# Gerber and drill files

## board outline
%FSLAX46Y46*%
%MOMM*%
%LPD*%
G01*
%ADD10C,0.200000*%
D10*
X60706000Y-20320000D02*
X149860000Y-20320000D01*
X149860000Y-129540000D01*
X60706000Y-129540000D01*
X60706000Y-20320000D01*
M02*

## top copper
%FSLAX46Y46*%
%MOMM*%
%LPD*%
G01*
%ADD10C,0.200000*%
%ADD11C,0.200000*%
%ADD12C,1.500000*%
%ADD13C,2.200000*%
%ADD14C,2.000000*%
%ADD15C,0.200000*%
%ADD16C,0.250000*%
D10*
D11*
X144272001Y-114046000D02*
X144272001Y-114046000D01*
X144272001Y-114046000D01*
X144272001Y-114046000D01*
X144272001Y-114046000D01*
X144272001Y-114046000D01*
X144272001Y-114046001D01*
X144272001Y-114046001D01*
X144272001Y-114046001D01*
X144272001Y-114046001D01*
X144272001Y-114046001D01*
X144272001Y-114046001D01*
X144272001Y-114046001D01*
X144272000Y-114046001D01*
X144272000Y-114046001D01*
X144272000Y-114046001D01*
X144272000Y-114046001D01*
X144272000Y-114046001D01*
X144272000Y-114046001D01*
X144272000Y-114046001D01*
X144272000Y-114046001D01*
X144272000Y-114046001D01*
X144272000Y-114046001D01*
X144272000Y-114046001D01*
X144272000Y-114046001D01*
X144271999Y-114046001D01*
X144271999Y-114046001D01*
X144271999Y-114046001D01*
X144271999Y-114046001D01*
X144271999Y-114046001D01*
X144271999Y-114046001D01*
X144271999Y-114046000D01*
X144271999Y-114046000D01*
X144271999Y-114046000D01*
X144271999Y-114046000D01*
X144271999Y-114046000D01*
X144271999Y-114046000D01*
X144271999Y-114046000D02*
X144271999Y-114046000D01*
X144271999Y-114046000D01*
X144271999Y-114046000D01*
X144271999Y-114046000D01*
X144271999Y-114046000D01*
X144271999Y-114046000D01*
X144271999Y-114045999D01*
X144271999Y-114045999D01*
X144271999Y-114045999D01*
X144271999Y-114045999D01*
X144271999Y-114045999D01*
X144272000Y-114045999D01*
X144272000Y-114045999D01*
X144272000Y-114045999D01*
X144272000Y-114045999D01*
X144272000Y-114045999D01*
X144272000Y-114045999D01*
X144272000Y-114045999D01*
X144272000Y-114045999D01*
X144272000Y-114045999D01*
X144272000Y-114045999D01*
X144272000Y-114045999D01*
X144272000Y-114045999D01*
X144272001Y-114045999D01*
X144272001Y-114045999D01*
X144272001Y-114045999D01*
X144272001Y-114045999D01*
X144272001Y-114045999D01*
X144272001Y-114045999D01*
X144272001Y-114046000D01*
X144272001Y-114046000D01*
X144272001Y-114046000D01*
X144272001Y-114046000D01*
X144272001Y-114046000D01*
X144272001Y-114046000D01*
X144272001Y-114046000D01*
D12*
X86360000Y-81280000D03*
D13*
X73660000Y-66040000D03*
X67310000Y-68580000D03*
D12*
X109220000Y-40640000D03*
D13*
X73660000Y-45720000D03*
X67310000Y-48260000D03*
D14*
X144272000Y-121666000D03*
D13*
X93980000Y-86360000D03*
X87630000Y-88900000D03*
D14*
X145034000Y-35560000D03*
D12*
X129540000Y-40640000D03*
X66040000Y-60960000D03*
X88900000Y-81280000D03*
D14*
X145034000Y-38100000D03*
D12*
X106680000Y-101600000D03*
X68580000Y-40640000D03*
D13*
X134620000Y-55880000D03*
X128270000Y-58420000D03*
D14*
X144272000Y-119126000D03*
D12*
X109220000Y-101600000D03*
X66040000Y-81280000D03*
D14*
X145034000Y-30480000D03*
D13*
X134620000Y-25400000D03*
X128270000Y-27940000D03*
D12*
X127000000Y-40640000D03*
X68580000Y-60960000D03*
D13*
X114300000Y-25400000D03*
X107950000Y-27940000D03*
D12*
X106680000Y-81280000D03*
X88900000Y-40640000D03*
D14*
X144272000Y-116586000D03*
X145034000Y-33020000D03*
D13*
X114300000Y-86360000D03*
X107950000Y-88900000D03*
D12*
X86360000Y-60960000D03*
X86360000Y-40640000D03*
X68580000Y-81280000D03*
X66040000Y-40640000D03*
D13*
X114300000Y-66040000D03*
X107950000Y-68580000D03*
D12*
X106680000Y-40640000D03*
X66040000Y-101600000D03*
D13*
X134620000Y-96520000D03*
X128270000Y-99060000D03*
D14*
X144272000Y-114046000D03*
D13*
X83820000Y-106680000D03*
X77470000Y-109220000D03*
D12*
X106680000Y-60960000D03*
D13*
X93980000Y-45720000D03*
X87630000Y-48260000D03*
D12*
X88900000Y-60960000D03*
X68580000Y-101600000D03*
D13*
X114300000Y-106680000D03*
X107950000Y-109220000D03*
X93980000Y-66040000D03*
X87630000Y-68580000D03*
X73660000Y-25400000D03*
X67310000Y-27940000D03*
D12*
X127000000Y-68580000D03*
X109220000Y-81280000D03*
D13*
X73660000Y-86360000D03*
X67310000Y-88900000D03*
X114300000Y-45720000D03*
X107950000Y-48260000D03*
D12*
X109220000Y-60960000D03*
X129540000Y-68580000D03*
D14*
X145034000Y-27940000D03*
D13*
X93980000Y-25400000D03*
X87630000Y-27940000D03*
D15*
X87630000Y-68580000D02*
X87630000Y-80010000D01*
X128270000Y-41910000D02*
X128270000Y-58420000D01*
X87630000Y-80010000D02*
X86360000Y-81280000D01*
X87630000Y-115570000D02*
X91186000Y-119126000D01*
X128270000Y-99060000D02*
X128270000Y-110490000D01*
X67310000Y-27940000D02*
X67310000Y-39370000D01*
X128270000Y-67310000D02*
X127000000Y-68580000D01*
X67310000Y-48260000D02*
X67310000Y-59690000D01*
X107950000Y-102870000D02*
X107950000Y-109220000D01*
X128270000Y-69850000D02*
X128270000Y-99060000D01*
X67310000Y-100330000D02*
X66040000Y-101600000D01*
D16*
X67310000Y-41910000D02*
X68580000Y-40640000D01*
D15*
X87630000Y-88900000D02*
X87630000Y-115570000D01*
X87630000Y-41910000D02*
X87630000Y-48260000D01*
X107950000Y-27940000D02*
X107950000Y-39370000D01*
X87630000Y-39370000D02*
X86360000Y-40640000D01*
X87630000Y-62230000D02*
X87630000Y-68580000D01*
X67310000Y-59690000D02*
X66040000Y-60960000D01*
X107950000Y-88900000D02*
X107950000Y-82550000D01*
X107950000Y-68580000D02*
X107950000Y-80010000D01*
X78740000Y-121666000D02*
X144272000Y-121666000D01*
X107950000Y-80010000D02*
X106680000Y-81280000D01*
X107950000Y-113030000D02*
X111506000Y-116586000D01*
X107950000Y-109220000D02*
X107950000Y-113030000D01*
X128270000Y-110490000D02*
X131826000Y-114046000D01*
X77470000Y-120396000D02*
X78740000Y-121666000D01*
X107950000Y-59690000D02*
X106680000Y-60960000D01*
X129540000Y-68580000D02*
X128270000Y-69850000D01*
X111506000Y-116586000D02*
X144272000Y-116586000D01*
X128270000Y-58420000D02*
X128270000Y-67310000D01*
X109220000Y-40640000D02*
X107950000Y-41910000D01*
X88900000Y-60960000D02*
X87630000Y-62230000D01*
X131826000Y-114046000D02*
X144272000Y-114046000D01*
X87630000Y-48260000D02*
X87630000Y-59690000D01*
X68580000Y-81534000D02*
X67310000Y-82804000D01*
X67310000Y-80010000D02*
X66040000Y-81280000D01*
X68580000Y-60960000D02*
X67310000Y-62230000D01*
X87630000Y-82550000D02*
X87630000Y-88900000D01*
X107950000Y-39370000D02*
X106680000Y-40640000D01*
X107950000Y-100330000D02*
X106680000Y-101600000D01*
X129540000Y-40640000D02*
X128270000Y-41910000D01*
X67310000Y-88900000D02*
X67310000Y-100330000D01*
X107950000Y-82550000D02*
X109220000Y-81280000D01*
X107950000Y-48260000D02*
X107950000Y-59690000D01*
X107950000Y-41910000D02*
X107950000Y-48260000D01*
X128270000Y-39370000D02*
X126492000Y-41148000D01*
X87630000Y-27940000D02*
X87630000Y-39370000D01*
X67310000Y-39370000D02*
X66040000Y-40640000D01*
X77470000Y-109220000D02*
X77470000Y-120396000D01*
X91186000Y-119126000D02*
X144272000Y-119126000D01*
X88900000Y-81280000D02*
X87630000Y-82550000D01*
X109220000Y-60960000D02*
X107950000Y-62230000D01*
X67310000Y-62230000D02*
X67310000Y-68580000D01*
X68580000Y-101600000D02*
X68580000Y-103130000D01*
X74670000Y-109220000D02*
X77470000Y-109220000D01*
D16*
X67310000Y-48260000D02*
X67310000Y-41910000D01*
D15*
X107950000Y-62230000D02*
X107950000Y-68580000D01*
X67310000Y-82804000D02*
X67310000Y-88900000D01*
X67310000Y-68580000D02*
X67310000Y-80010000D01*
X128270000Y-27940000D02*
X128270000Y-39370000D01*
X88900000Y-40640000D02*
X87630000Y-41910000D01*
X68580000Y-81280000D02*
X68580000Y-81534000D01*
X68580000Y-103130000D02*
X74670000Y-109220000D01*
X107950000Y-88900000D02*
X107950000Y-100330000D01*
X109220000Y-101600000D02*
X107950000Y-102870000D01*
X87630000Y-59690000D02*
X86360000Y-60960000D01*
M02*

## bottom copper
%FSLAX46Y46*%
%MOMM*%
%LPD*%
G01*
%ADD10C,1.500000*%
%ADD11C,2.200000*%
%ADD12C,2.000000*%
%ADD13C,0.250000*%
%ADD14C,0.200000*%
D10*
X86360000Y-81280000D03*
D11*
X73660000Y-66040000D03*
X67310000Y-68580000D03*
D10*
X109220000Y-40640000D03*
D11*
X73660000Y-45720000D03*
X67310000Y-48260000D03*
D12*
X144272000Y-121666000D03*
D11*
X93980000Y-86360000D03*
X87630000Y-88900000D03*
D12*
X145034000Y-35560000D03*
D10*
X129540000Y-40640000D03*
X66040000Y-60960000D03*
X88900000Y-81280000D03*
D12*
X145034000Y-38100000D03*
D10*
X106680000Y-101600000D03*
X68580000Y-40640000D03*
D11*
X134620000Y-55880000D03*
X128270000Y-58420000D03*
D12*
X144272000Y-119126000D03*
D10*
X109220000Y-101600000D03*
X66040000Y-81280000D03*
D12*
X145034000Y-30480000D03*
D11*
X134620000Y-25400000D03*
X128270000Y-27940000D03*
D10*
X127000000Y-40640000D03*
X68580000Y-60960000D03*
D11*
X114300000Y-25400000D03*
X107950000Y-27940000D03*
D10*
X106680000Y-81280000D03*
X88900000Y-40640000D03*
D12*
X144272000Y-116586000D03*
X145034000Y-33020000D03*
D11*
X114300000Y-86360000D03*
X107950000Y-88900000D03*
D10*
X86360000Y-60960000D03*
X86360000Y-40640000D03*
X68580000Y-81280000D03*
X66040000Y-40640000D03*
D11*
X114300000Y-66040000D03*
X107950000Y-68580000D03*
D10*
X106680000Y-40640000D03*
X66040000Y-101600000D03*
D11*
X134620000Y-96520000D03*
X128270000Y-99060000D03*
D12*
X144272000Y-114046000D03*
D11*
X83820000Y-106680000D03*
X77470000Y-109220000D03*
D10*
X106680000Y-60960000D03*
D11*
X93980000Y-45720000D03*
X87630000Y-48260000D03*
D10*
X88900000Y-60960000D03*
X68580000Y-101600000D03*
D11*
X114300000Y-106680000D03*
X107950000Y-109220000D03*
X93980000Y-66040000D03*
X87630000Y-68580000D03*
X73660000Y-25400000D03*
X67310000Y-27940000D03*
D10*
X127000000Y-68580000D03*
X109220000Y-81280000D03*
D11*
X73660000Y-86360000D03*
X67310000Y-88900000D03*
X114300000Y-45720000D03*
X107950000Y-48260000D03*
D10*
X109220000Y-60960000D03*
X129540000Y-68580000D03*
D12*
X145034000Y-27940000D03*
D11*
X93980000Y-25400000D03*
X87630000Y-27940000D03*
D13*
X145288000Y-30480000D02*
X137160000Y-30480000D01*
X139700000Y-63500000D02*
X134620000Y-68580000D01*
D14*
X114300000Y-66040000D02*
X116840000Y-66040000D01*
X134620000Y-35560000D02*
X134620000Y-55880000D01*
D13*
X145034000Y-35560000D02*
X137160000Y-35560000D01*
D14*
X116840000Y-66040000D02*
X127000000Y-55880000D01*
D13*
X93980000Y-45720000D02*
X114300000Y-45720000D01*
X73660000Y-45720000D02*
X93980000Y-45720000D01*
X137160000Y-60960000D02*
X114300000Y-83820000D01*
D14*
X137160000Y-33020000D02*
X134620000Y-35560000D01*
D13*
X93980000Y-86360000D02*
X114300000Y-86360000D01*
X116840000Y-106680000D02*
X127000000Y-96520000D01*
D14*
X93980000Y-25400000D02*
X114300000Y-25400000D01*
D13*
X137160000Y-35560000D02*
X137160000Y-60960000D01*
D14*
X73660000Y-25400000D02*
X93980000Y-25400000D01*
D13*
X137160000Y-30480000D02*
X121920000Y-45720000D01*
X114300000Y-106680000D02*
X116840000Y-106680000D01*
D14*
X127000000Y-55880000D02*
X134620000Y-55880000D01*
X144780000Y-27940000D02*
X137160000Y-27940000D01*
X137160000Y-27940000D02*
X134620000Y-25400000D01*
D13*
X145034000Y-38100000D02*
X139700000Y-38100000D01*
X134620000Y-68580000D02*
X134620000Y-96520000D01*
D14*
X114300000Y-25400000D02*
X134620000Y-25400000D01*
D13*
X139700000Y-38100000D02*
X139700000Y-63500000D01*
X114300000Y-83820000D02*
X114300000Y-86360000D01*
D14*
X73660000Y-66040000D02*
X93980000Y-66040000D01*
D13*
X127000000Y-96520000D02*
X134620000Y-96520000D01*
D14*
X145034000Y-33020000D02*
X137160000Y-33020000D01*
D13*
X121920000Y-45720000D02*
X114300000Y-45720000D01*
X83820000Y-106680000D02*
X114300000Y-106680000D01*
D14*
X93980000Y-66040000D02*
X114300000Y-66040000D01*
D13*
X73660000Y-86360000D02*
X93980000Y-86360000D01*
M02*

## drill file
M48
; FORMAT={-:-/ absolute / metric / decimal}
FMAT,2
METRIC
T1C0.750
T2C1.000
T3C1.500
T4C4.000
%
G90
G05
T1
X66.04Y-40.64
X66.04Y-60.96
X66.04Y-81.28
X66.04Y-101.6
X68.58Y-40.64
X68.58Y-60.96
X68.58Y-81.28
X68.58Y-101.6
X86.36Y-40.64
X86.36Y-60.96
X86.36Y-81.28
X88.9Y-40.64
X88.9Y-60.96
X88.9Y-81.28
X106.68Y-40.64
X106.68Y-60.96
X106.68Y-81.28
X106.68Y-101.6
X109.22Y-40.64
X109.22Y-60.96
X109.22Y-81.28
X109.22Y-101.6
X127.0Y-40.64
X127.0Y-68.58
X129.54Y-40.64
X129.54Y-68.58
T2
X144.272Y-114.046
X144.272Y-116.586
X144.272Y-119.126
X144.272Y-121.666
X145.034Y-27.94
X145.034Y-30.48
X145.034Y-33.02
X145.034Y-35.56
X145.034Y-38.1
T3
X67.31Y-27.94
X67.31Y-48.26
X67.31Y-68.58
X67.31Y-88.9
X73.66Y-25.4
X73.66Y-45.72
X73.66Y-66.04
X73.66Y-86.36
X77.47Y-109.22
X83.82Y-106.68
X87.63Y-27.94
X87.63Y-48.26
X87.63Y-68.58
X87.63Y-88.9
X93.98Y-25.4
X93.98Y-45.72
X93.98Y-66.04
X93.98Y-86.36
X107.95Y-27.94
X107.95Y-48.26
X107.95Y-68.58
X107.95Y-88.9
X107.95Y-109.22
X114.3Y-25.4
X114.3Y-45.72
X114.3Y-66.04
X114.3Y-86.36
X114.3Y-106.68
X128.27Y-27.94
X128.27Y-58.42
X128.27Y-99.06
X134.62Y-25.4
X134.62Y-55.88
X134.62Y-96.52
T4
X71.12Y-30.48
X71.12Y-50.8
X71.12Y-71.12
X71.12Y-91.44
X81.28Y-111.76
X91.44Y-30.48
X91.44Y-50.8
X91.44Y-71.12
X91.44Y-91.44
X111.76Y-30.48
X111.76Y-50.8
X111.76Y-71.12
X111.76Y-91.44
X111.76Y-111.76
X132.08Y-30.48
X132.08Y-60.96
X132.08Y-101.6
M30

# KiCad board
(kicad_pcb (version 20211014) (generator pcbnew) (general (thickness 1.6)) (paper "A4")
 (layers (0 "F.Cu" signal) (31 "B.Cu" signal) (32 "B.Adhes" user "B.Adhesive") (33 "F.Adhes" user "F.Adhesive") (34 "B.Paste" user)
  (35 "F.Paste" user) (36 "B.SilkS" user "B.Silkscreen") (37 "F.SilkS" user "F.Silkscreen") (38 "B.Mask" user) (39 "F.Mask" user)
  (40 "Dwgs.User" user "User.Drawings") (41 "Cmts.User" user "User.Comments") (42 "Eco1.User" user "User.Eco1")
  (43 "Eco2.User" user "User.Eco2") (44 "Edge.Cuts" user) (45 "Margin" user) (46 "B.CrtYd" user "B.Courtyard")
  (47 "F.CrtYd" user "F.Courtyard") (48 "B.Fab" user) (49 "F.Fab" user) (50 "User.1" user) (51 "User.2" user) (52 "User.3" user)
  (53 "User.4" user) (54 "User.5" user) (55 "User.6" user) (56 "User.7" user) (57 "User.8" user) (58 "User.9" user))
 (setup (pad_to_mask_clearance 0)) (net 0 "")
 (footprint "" (layer "F.Cu") (at 86.36 81.28)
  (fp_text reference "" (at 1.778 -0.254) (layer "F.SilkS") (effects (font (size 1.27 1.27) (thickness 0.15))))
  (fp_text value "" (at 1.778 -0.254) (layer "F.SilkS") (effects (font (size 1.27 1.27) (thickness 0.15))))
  (pad "1" thru_hole circle (at 0 0) (size 1.5 1.5) (drill 0.75) (layers *.Cu *.Mask)))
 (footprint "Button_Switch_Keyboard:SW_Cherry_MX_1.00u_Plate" (layer "F.Cu") (at 73.66 66.04)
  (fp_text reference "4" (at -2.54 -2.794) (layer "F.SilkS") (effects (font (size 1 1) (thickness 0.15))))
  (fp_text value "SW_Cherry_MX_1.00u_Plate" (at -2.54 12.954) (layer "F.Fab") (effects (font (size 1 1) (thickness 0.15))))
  (pad "" np_thru_hole circle (at -2.54 5.08) (size 4 4) (drill 4) (layers *.Cu *.Mask))
  (pad "1" thru_hole circle (at 0 0) (size 2.2 2.2) (drill 1.5) (layers *.Cu *.Mask))
  (pad "2" thru_hole circle (at -6.35 2.54) (size 2.2 2.2) (drill 1.5) (layers *.Cu *.Mask)))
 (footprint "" (layer "F.Cu") (at 109.22 40.64)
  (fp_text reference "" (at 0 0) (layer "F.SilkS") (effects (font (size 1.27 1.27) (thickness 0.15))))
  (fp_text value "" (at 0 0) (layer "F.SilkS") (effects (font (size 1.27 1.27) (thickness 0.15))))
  (pad "1" thru_hole circle (at 0 0) (size 1.5 1.5) (drill 0.75) (layers *.Cu *.Mask)))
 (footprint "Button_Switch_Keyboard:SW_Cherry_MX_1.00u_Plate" (layer "F.Cu") (at 73.66 45.72)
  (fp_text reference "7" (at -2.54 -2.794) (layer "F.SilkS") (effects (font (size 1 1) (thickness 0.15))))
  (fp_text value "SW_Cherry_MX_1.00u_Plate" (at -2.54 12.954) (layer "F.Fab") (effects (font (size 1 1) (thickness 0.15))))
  (pad "" np_thru_hole circle (at -2.54 5.08) (size 4 4) (drill 4) (layers *.Cu *.Mask))
  (pad "1" thru_hole circle (at 0 0) (size 2.2 2.2) (drill 1.5) (layers *.Cu *.Mask))
  (pad "2" thru_hole circle (at -6.35 2.54) (size 2.2 2.2) (drill 1.5) (layers *.Cu *.Mask)))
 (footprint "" (layer "F.Cu") (at 144.272 121.666)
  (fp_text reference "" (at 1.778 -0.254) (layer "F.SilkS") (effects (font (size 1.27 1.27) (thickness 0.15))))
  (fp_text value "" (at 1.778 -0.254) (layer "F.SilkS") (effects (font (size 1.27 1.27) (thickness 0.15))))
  (pad "1" thru_hole circle (at 0 0) (size 2 2) (drill 1) (layers *.Cu *.Mask)))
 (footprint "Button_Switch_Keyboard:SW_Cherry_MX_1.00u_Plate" (layer "F.Cu") (at 93.98 86.36)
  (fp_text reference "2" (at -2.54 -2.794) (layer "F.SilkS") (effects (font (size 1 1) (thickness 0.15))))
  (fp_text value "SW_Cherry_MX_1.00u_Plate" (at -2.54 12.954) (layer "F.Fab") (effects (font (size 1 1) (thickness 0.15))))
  (pad "" np_thru_hole circle (at -2.54 5.08) (size 4 4) (drill 4) (layers *.Cu *.Mask))
  (pad "1" thru_hole circle (at 0 0) (size 2.2 2.2) (drill 1.5) (layers *.Cu *.Mask))
  (pad "2" thru_hole circle (at -6.35 2.54) (size 2.2 2.2) (drill 1.5) (layers *.Cu *.Mask)))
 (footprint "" (layer "F.Cu") (at 145.034 35.56)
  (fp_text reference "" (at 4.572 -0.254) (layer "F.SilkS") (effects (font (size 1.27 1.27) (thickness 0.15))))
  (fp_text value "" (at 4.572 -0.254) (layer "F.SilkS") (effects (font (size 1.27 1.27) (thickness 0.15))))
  (pad "1" thru_hole circle (at 0 0) (size 2 2) (drill 1) (layers *.Cu *.Mask)))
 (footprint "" (layer "F.Cu") (at 129.54 40.64)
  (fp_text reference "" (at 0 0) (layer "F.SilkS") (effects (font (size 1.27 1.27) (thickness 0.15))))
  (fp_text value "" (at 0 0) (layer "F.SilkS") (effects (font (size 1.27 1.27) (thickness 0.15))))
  (pad "1" thru_hole circle (at 0 0) (size 1.5 1.5) (drill 0.75) (layers *.Cu *.Mask)))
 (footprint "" (layer "F.Cu") (at 66.04 60.96)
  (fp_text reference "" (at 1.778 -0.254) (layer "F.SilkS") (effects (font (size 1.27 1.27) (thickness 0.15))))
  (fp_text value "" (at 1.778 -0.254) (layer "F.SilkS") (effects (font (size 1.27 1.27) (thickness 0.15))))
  (pad "1" thru_hole circle (at 0 0) (size 1.5 1.5) (drill 0.75) (layers *.Cu *.Mask)))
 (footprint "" (layer "F.Cu") (at 88.9 81.28)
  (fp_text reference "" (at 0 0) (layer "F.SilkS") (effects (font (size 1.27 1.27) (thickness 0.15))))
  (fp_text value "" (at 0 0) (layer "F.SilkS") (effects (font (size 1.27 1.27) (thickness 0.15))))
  (pad "1" thru_hole circle (at 0 0) (size 1.5 1.5) (drill 0.75) (layers *.Cu *.Mask)))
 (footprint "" (layer "F.Cu") (at 145.034 38.1)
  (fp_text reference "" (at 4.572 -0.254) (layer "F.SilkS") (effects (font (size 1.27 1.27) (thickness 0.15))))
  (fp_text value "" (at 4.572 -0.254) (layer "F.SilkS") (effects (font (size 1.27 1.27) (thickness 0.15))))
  (pad "1" thru_hole circle (at 0 0) (size 2 2) (drill 1) (layers *.Cu *.Mask)))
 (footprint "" (layer "F.Cu") (at 106.68 101.6)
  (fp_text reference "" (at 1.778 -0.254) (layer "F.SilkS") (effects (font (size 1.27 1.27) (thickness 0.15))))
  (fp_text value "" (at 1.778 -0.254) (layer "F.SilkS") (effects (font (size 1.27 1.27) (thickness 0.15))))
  (pad "1" thru_hole circle (at 0 0) (size 1.5 1.5) (drill 0.75) (layers *.Cu *.Mask)))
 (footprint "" (layer "F.Cu") (at 68.58 40.64)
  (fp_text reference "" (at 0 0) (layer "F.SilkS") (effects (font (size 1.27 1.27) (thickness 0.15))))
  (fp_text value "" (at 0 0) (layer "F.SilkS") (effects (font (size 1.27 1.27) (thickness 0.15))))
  (pad "1" thru_hole circle (at 0 0) (size 1.5 1.5) (drill 0.75) (layers *.Cu *.Mask)))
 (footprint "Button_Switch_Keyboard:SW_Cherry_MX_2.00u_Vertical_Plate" (layer "F.Cu") (at 134.62 55.88)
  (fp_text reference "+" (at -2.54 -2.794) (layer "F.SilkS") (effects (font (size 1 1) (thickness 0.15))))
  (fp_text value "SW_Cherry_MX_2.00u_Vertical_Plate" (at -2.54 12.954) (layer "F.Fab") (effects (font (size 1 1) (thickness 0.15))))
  (pad "" np_thru_hole circle (at -2.54 5.08) (size 4 4) (drill 4) (layers *.Cu *.Mask))
  (pad "1" thru_hole circle (at 0 0) (size 2.2 2.2) (drill 1.5) (layers *.Cu *.Mask))
  (pad "2" thru_hole circle (at -6.35 2.54) (size 2.2 2.2) (drill 1.5) (layers *.Cu *.Mask)))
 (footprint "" (layer "F.Cu") (at 144.272 119.126)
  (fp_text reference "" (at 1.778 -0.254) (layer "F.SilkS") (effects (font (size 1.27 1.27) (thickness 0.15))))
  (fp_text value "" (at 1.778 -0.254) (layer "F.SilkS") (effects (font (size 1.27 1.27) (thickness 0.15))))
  (pad "1" thru_hole circle (at 0 0) (size 2 2) (drill 1) (layers *.Cu *.Mask)))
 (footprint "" (layer "F.Cu") (at 109.22 101.6)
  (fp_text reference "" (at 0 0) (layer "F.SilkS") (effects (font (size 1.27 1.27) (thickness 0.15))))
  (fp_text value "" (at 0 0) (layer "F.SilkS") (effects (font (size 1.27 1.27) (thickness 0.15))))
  (pad "1" thru_hole circle (at 0 0) (size 1.5 1.5) (drill 0.75) (layers *.Cu *.Mask)))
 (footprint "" (layer "F.Cu") (at 66.04 81.28)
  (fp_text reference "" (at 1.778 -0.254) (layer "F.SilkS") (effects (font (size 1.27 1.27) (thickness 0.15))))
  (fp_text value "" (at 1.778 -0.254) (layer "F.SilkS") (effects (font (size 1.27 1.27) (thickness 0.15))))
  (pad "1" thru_hole circle (at 0 0) (size 1.5 1.5) (drill 0.75) (layers *.Cu *.Mask)))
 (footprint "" (layer "F.Cu") (at 145.034 30.48)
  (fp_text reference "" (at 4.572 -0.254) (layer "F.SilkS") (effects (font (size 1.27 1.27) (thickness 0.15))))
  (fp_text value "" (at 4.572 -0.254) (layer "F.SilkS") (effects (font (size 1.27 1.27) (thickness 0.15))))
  (pad "1" thru_hole circle (at 0 0) (size 2 2) (drill 1) (layers *.Cu *.Mask)))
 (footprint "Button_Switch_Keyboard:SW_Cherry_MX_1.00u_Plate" (layer "F.Cu") (at 134.62 25.4)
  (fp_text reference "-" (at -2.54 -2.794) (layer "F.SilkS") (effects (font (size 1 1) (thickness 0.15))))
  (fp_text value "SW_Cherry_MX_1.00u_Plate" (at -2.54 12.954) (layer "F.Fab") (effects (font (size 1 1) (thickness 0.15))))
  (pad "" np_thru_hole circle (at -2.54 5.08) (size 4 4) (drill 4) (layers *.Cu *.Mask))
  (pad "1" thru_hole circle (at 0 0) (size 2.2 2.2) (drill 1.5) (layers *.Cu *.Mask))
  (pad "2" thru_hole circle (at -6.35 2.54) (size 2.2 2.2) (drill 1.5) (layers *.Cu *.Mask)))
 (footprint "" (layer "F.Cu") (at 127 40.64)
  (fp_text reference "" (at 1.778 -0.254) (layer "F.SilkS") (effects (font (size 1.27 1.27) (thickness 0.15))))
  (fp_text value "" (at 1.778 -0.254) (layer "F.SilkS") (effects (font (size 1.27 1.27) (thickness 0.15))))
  (pad "1" thru_hole circle (at 0 0) (size 1.5 1.5) (drill 0.75) (layers *.Cu *.Mask)))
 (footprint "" (layer "F.Cu") (at 68.58 60.96)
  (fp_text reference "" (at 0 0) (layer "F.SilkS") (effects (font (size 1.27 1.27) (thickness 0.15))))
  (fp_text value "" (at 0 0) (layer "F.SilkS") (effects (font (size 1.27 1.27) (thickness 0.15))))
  (pad "1" thru_hole circle (at 0 0) (size 1.5 1.5) (drill 0.75) (layers *.Cu *.Mask)))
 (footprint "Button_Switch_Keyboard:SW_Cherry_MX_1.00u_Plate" (layer "F.Cu") (at 114.3 25.4)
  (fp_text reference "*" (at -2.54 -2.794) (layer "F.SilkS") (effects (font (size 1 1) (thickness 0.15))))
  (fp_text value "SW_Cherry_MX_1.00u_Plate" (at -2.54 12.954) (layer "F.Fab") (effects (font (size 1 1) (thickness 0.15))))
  (pad "" np_thru_hole circle (at -2.54 5.08) (size 4 4) (drill 4) (layers *.Cu *.Mask))
  (pad "1" thru_hole circle (at 0 0) (size 2.2 2.2) (drill 1.5) (layers *.Cu *.Mask))
  (pad "2" thru_hole circle (at -6.35 2.54) (size 2.2 2.2) (drill 1.5) (layers *.Cu *.Mask)))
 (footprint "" (layer "F.Cu") (at 106.68 81.28)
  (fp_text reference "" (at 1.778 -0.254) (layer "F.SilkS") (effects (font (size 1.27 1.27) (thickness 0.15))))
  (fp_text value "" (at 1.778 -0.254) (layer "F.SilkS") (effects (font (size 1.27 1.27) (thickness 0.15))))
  (pad "1" thru_hole circle (at 0 0) (size 1.5 1.5) (drill 0.75) (layers *.Cu *.Mask)))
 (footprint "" (layer "F.Cu") (at 88.9 40.64)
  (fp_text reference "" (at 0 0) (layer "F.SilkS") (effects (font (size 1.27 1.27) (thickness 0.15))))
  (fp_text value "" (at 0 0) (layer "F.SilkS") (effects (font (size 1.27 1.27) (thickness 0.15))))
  (pad "1" thru_hole circle (at 0 0) (size 1.5 1.5) (drill 0.75) (layers *.Cu *.Mask)))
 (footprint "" (layer "F.Cu") (at 144.272 116.586)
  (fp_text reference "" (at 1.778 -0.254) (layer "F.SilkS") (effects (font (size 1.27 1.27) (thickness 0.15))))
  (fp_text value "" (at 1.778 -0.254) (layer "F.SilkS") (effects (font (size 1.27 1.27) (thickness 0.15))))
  (pad "1" thru_hole circle (at 0 0) (size 2 2) (drill 1) (layers *.Cu *.Mask)))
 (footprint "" (layer "F.Cu") (at 145.034 33.02)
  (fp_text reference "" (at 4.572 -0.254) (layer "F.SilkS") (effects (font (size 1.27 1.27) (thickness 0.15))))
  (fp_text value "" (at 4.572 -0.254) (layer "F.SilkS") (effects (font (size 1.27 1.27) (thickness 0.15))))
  (pad "1" thru_hole circle (at 0 0) (size 2 2) (drill 1) (layers *.Cu *.Mask)))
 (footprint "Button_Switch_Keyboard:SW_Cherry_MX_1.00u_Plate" (layer "F.Cu") (at 114.3 86.36)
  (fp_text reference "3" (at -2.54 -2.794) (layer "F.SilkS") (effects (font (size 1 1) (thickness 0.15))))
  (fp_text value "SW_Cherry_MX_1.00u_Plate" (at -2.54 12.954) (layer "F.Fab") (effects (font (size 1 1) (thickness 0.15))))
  (pad "" np_thru_hole circle (at -2.54 5.08) (size 4 4) (drill 4) (layers *.Cu *.Mask))
  (pad "1" thru_hole circle (at 0 0) (size 2.2 2.2) (drill 1.5) (layers *.Cu *.Mask))
  (pad "2" thru_hole circle (at -6.35 2.54) (size 2.2 2.2) (drill 1.5) (layers *.Cu *.Mask)))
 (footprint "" (layer "F.Cu") (at 86.36 60.96)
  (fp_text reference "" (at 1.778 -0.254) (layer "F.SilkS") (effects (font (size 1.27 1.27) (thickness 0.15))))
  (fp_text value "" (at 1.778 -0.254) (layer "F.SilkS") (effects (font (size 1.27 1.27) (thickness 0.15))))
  (pad "1" thru_hole circle (at 0 0) (size 1.5 1.5) (drill 0.75) (layers *.Cu *.Mask)))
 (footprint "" (layer "F.Cu") (at 86.36 40.64)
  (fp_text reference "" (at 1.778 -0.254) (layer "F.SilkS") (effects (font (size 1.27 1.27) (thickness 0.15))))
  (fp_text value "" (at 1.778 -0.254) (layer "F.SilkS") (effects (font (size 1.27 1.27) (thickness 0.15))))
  (pad "1" thru_hole circle (at 0 0) (size 1.5 1.5) (drill 0.75) (layers *.Cu *.Mask)))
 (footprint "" (layer "F.Cu") (at 68.58 81.28)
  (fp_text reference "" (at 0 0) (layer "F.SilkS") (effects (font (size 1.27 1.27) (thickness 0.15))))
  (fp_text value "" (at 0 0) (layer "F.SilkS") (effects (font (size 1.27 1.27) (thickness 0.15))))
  (pad "1" thru_hole circle (at 0 0) (size 1.5 1.5) (drill 0.75) (layers *.Cu *.Mask)))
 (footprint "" (layer "F.Cu") (at 66.04 40.64)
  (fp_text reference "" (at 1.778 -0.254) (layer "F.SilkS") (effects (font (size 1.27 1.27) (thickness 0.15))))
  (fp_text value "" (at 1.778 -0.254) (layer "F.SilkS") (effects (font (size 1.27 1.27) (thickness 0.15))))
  (pad "1" thru_hole circle (at 0 0) (size 1.5 1.5) (drill 0.75) (layers *.Cu *.Mask)))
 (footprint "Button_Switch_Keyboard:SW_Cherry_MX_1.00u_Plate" (layer "F.Cu") (at 114.3 66.04)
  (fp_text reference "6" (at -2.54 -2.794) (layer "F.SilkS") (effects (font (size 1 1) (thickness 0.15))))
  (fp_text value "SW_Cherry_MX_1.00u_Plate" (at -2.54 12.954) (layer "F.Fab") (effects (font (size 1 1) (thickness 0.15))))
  (pad "" np_thru_hole circle (at -2.54 5.08) (size 4 4) (drill 4) (layers *.Cu *.Mask))
  (pad "1" thru_hole circle (at 0 0) (size 2.2 2.2) (drill 1.5) (layers *.Cu *.Mask))
  (pad "2" thru_hole circle (at -6.35 2.54) (size 2.2 2.2) (drill 1.5) (layers *.Cu *.Mask)))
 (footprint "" (layer "F.Cu") (at 106.68 40.64)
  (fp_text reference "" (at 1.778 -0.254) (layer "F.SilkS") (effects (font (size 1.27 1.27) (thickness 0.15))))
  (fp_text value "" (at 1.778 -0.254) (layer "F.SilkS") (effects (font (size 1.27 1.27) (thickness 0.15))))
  (pad "1" thru_hole circle (at 0 0) (size 1.5 1.5) (drill 0.75) (layers *.Cu *.Mask)))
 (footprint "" (layer "F.Cu") (at 66.04 101.6)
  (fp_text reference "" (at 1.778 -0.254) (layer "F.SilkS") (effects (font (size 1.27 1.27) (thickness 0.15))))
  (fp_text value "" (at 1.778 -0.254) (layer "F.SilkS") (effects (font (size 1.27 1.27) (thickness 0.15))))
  (pad "1" thru_hole circle (at 0 0) (size 1.5 1.5) (drill 0.75) (layers *.Cu *.Mask)))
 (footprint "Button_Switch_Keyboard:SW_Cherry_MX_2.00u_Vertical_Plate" (layer "F.Cu") (at 134.62 96.52)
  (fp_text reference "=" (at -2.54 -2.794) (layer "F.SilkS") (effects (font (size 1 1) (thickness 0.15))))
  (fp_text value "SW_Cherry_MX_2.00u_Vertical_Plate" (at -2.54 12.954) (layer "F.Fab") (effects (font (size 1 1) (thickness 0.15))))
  (pad "" np_thru_hole circle (at -2.54 5.08) (size 4 4) (drill 4) (layers *.Cu *.Mask))
  (pad "1" thru_hole circle (at 0 0) (size 2.2 2.2) (drill 1.5) (layers *.Cu *.Mask))
  (pad "2" thru_hole circle (at -6.35 2.54) (size 2.2 2.2) (drill 1.5) (layers *.Cu *.Mask)))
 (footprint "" (layer "F.Cu") (at 144.272 114.046)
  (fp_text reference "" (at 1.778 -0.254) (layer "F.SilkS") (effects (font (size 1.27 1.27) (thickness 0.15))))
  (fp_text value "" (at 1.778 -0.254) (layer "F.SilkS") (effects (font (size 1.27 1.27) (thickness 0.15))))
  (pad "1" thru_hole circle (at 0 0) (size 2 2) (drill 1) (layers *.Cu *.Mask)))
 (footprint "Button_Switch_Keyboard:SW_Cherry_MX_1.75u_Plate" (layer "F.Cu") (at 83.82 106.68)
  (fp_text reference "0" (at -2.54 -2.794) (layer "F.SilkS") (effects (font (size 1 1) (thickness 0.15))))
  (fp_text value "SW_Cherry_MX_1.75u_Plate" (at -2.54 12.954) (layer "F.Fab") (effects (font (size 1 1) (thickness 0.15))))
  (pad "" np_thru_hole circle (at -2.54 5.08) (size 4 4) (drill 4) (layers *.Cu *.Mask))
  (pad "1" thru_hole circle (at 0 0) (size 2.2 2.2) (drill 1.5) (layers *.Cu *.Mask))
  (pad "2" thru_hole circle (at -6.35 2.54) (size 2.2 2.2) (drill 1.5) (layers *.Cu *.Mask)))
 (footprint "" (layer "F.Cu") (at 106.68 60.96)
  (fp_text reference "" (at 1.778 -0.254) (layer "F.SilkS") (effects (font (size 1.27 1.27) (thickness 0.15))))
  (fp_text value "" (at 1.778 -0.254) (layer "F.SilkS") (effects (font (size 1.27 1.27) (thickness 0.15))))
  (pad "1" thru_hole circle (at 0 0) (size 1.5 1.5) (drill 0.75) (layers *.Cu *.Mask)))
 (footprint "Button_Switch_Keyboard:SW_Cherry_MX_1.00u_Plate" (layer "F.Cu") (at 93.98 45.72)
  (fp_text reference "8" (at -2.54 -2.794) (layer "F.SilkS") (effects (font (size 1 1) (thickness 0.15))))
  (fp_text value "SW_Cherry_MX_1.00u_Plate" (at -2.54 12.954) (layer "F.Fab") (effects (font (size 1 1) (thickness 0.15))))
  (pad "" np_thru_hole circle (at -2.54 5.08) (size 4 4) (drill 4) (layers *.Cu *.Mask))
  (pad "1" thru_hole circle (at 0 0) (size 2.2 2.2) (drill 1.5) (layers *.Cu *.Mask))
  (pad "2" thru_hole circle (at -6.35 2.54) (size 2.2 2.2) (drill 1.5) (layers *.Cu *.Mask)))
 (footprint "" (layer "F.Cu") (at 88.9 60.96)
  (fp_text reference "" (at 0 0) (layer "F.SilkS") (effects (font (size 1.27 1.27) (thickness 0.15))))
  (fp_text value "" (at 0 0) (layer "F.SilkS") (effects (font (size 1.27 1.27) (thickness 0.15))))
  (pad "1" thru_hole circle (at 0 0) (size 1.5 1.5) (drill 0.75) (layers *.Cu *.Mask)))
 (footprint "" (layer "F.Cu") (at 68.58 101.6)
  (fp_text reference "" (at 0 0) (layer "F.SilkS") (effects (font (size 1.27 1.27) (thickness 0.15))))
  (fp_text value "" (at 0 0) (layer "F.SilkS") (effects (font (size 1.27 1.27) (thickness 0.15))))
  (pad "1" thru_hole circle (at 0 0) (size 1.5 1.5) (drill 0.75) (layers *.Cu *.Mask)))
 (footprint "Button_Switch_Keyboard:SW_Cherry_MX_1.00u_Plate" (layer "F.Cu") (at 114.3 106.68)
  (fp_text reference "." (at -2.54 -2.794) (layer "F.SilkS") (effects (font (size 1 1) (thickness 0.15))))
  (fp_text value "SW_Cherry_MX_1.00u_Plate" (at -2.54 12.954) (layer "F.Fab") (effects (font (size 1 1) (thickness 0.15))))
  (pad "" np_thru_hole circle (at -2.54 5.08) (size 4 4) (drill 4) (layers *.Cu *.Mask))
  (pad "1" thru_hole circle (at 0 0) (size 2.2 2.2) (drill 1.5) (layers *.Cu *.Mask))
  (pad "2" thru_hole circle (at -6.35 2.54) (size 2.2 2.2) (drill 1.5) (layers *.Cu *.Mask)))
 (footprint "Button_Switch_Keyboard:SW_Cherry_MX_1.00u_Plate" (layer "F.Cu") (at 93.98 66.04)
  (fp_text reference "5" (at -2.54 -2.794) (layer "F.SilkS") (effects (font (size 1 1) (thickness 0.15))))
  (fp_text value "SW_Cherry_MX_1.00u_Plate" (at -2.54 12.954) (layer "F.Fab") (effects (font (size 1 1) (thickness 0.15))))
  (pad "" np_thru_hole circle (at -2.54 5.08) (size 4 4) (drill 4) (layers *.Cu *.Mask))
  (pad "1" thru_hole circle (at 0 0) (size 2.2 2.2) (drill 1.5) (layers *.Cu *.Mask))
  (pad "2" thru_hole circle (at -6.35 2.54) (size 2.2 2.2) (drill 1.5) (layers *.Cu *.Mask)))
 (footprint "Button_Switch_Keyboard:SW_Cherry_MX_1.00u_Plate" (layer "F.Cu") (at 73.66 25.4)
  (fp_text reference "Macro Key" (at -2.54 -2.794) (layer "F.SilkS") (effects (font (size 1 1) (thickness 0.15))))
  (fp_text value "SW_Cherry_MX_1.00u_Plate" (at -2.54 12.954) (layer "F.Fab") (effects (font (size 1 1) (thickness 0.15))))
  (pad "" np_thru_hole circle (at -2.54 5.08) (size 4 4) (drill 4) (layers *.Cu *.Mask))
  (pad "1" thru_hole circle (at 0 0) (size 2.2 2.2) (drill 1.5) (layers *.Cu *.Mask))
  (pad "2" thru_hole circle (at -6.35 2.54) (size 2.2 2.2) (drill 1.5) (layers *.Cu *.Mask)))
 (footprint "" (layer "F.Cu") (at 127 68.58)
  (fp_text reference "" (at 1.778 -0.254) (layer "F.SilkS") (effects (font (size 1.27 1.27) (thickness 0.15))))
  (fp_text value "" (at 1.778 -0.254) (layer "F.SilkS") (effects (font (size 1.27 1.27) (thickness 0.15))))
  (pad "1" thru_hole circle (at 0 0) (size 1.5 1.5) (drill 0.75) (layers *.Cu *.Mask)))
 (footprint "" (layer "F.Cu") (at 109.22 81.28)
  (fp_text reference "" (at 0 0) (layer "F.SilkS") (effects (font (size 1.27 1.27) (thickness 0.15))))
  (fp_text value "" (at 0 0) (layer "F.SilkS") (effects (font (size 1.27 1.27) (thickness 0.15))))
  (pad "1" thru_hole circle (at 0 0) (size 1.5 1.5) (drill 0.75) (layers *.Cu *.Mask)))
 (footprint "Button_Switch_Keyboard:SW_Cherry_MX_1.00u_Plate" (layer "F.Cu") (at 73.66 86.36)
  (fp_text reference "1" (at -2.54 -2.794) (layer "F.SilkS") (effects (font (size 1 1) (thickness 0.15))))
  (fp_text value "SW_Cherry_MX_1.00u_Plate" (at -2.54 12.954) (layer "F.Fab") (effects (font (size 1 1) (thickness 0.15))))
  (pad "" np_thru_hole circle (at -2.54 5.08) (size 4 4) (drill 4) (layers *.Cu *.Mask))
  (pad "1" thru_hole circle (at 0 0) (size 2.2 2.2) (drill 1.5) (layers *.Cu *.Mask))
  (pad "2" thru_hole circle (at -6.35 2.54) (size 2.2 2.2) (drill 1.5) (layers *.Cu *.Mask)))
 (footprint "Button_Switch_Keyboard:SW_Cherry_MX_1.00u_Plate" (layer "F.Cu") (at 114.3 45.72)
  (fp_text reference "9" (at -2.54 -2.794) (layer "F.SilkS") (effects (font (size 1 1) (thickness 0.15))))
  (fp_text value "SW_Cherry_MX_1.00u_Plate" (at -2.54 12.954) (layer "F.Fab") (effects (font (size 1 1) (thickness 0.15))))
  (pad "" np_thru_hole circle (at -2.54 5.08) (size 4 4) (drill 4) (layers *.Cu *.Mask))
  (pad "1" thru_hole circle (at 0 0) (size 2.2 2.2) (drill 1.5) (layers *.Cu *.Mask))
  (pad "2" thru_hole circle (at -6.35 2.54) (size 2.2 2.2) (drill 1.5) (layers *.Cu *.Mask)))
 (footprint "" (layer "F.Cu") (at 109.22 60.96)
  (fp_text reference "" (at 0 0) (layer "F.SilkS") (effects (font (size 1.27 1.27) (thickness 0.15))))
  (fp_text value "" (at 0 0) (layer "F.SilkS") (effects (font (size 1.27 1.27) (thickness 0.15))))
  (pad "1" thru_hole circle (at 0 0) (size 1.5 1.5) (drill 0.75) (layers *.Cu *.Mask)))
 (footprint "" (layer "F.Cu") (at 129.54 68.58)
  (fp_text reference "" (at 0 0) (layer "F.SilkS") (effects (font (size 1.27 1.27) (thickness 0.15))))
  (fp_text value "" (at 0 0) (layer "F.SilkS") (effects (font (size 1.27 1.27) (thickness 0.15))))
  (pad "1" thru_hole circle (at 0 0) (size 1.5 1.5) (drill 0.75) (layers *.Cu *.Mask)))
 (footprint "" (layer "F.Cu") (at 145.034 27.94)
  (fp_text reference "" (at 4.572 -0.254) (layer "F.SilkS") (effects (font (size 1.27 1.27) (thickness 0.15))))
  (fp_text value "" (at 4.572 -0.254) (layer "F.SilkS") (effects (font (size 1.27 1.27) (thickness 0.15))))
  (pad "1" thru_hole circle (at 0 0) (size 2 2) (drill 1) (layers *.Cu *.Mask)))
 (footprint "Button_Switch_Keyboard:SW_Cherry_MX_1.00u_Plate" (layer "F.Cu") (at 93.98 25.4)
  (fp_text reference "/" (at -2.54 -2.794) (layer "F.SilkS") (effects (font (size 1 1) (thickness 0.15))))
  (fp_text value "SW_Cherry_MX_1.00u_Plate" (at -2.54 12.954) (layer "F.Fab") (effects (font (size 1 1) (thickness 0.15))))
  (pad "" np_thru_hole circle (at -2.54 5.08) (size 4 4) (drill 4) (layers *.Cu *.Mask))
  (pad "1" thru_hole circle (at 0 0) (size 2.2 2.2) (drill 1.5) (layers *.Cu *.Mask))
  (pad "2" thru_hole circle (at -6.35 2.54) (size 2.2 2.2) (drill 1.5) (layers *.Cu *.Mask)))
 (gr_circle (center 144.272 114.046) (end 144.272 114.046) (layer "F.Cu") (width 0.2) (fill none))
 (gr_rect (start 149.86 20.32) (end 60.706 129.54) (layer "Edge.Cuts") (width 0.2) (fill none))
 (segment (start 87.63 68.58) (end 87.63 80.01) (width 0.2) (layer "F.Cu") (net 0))
 (segment (start 128.27 41.91) (end 128.27 58.42) (width 0.2) (layer "F.Cu") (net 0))
 (segment (start 87.63 80.01) (end 86.36 81.28) (width 0.2) (layer "F.Cu") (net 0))
 (segment (start 87.63 115.57) (end 91.186 119.126) (width 0.2) (layer "F.Cu") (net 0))
 (segment (start 128.27 99.06) (end 128.27 110.49) (width 0.2) (layer "F.Cu") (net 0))
 (segment (start 67.31 27.94) (end 67.31 39.37) (width 0.2) (layer "F.Cu") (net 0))
 (segment (start 128.27 67.31) (end 127 68.58) (width 0.2) (layer "F.Cu") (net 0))
 (segment (start 67.31 48.26) (end 67.31 59.69) (width 0.2) (layer "F.Cu") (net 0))
 (segment (start 107.95 102.87) (end 107.95 109.22) (width 0.2) (layer "F.Cu") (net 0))
 (segment (start 128.27 69.85) (end 128.27 99.06) (width 0.2) (layer "F.Cu") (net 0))
 (segment (start 67.31 100.33) (end 66.04 101.6) (width 0.2) (layer "F.Cu") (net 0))
 (segment (start 67.31 41.91) (end 68.58 40.64) (width 0.25) (layer "F.Cu") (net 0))
 (segment (start 87.63 88.9) (end 87.63 115.57) (width 0.2) (layer "F.Cu") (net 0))
 (segment (start 87.63 41.91) (end 87.63 48.26) (width 0.2) (layer "F.Cu") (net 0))
 (segment (start 107.95 27.94) (end 107.95 39.37) (width 0.2) (layer "F.Cu") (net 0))
 (segment (start 87.63 39.37) (end 86.36 40.64) (width 0.2) (layer "F.Cu") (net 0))
 (segment (start 87.63 62.23) (end 87.63 68.58) (width 0.2) (layer "F.Cu") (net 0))
 (segment (start 67.31 59.69) (end 66.04 60.96) (width 0.2) (layer "F.Cu") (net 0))
 (segment (start 107.95 88.9) (end 107.95 82.55) (width 0.2) (layer "F.Cu") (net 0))
 (segment (start 107.95 68.58) (end 107.95 80.01) (width 0.2) (layer "F.Cu") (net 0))
 (segment (start 78.74 121.666) (end 144.272 121.666) (width 0.2) (layer "F.Cu") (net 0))
 (segment (start 107.95 80.01) (end 106.68 81.28) (width 0.2) (layer "F.Cu") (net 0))
 (segment (start 107.95 113.03) (end 111.506 116.586) (width 0.2) (layer "F.Cu") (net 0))
 (segment (start 107.95 109.22) (end 107.95 113.03) (width 0.2) (layer "F.Cu") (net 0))
 (segment (start 128.27 110.49) (end 131.826 114.046) (width 0.2) (layer "F.Cu") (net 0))
 (segment (start 77.47 120.396) (end 78.74 121.666) (width 0.2) (layer "F.Cu") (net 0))
 (segment (start 107.95 59.69) (end 106.68 60.96) (width 0.2) (layer "F.Cu") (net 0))
 (segment (start 129.54 68.58) (end 128.27 69.85) (width 0.2) (layer "F.Cu") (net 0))
 (segment (start 111.506 116.586) (end 144.272 116.586) (width 0.2) (layer "F.Cu") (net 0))
 (segment (start 128.27 58.42) (end 128.27 67.31) (width 0.2) (layer "F.Cu") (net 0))
 (segment (start 109.22 40.64) (end 107.95 41.91) (width 0.2) (layer "F.Cu") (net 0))
 (segment (start 88.9 60.96) (end 87.63 62.23) (width 0.2) (layer "F.Cu") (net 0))
 (segment (start 131.826 114.046) (end 144.272 114.046) (width 0.2) (layer "F.Cu") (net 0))
 (segment (start 87.63 48.26) (end 87.63 59.69) (width 0.2) (layer "F.Cu") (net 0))
 (segment (start 68.58 81.534) (end 67.31 82.804) (width 0.2) (layer "F.Cu") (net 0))
 (segment (start 67.31 80.01) (end 66.04 81.28) (width 0.2) (layer "F.Cu") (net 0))
 (segment (start 68.58 60.96) (end 67.31 62.23) (width 0.2) (layer "F.Cu") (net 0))
 (segment (start 87.63 82.55) (end 87.63 88.9) (width 0.2) (layer "F.Cu") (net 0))
 (segment (start 107.95 39.37) (end 106.68 40.64) (width 0.2) (layer "F.Cu") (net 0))
 (segment (start 107.95 100.33) (end 106.68 101.6) (width 0.2) (layer "F.Cu") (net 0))
 (segment (start 129.54 40.64) (end 128.27 41.91) (width 0.2) (layer "F.Cu") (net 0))
 (segment (start 67.31 88.9) (end 67.31 100.33) (width 0.2) (layer "F.Cu") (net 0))
 (segment (start 107.95 82.55) (end 109.22 81.28) (width 0.2) (layer "F.Cu") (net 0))
 (segment (start 107.95 48.26) (end 107.95 59.69) (width 0.2) (layer "F.Cu") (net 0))
 (segment (start 107.95 41.91) (end 107.95 48.26) (width 0.2) (layer "F.Cu") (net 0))
 (segment (start 128.27 39.37) (end 126.492 41.148) (width 0.2) (layer "F.Cu") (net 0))
 (segment (start 87.63 27.94) (end 87.63 39.37) (width 0.2) (layer "F.Cu") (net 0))
 (segment (start 67.31 39.37) (end 66.04 40.64) (width 0.2) (layer "F.Cu") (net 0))
 (segment (start 77.47 109.22) (end 77.47 120.396) (width 0.2) (layer "F.Cu") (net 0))
 (segment (start 91.186 119.126) (end 144.272 119.126) (width 0.2) (layer "F.Cu") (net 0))
 (segment (start 88.9 81.28) (end 87.63 82.55) (width 0.2) (layer "F.Cu") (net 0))
 (segment (start 109.22 60.96) (end 107.95 62.23) (width 0.2) (layer "F.Cu") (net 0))
 (segment (start 67.31 62.23) (end 67.31 68.58) (width 0.2) (layer "F.Cu") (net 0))
 (segment (start 68.58 101.6) (end 68.58 103.13) (width 0.2) (layer "F.Cu") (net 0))
 (segment (start 74.67 109.22) (end 77.47 109.22) (width 0.2) (layer "F.Cu") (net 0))
 (segment (start 67.31 48.26) (end 67.31 41.91) (width 0.25) (layer "F.Cu") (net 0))
 (segment (start 107.95 62.23) (end 107.95 68.58) (width 0.2) (layer "F.Cu") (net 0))
 (segment (start 67.31 82.804) (end 67.31 88.9) (width 0.2) (layer "F.Cu") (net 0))
 (segment (start 67.31 68.58) (end 67.31 80.01) (width 0.2) (layer "F.Cu") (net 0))
 (segment (start 128.27 27.94) (end 128.27 39.37) (width 0.2) (layer "F.Cu") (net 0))
 (segment (start 88.9 40.64) (end 87.63 41.91) (width 0.2) (layer "F.Cu") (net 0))
 (segment (start 68.58 81.28) (end 68.58 81.534) (width 0.2) (layer "F.Cu") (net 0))
 (segment (start 68.58 103.13) (end 74.67 109.22) (width 0.2) (layer "F.Cu") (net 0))
 (segment (start 107.95 88.9) (end 107.95 100.33) (width 0.2) (layer "F.Cu") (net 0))
 (segment (start 109.22 101.6) (end 107.95 102.87) (width 0.2) (layer "F.Cu") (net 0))
 (segment (start 87.63 59.69) (end 86.36 60.96) (width 0.2) (layer "F.Cu") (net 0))
 (segment (start 145.288 30.48) (end 137.16 30.48) (width 0.25) (layer "B.Cu") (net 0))
 (segment (start 139.7 63.5) (end 134.62 68.58) (width 0.25) (layer "B.Cu") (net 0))
 (segment (start 114.3 66.04) (end 116.84 66.04) (width 0.2) (layer "B.Cu") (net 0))
 (segment (start 134.62 35.56) (end 134.62 55.88) (width 0.2) (layer "B.Cu") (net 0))
 (segment (start 145.034 35.56) (end 137.16 35.56) (width 0.25) (layer "B.Cu") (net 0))
 (segment (start 116.84 66.04) (end 127 55.88) (width 0.2) (layer "B.Cu") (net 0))
 (segment (start 93.98 45.72) (end 114.3 45.72) (width 0.25) (layer "B.Cu") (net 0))
 (segment (start 73.66 45.72) (end 93.98 45.72) (width 0.25) (layer "B.Cu") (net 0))
 (segment (start 137.16 60.96) (end 114.3 83.82) (width 0.25) (layer "B.Cu") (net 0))
 (segment (start 137.16 33.02) (end 134.62 35.56) (width 0.2) (layer "B.Cu") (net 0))
 (segment (start 93.98 86.36) (end 114.3 86.36) (width 0.25) (layer "B.Cu") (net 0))
 (segment (start 116.84 106.68) (end 127 96.52) (width 0.25) (layer "B.Cu") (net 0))
 (segment (start 93.98 25.4) (end 114.3 25.4) (width 0.2) (layer "B.Cu") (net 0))
 (segment (start 137.16 35.56) (end 137.16 60.96) (width 0.25) (layer "B.Cu") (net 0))
 (segment (start 73.66 25.4) (end 93.98 25.4) (width 0.2) (layer "B.Cu") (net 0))
 (segment (start 137.16 30.48) (end 121.92 45.72) (width 0.25) (layer "B.Cu") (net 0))
 (segment (start 114.3 106.68) (end 116.84 106.68) (width 0.25) (layer "B.Cu") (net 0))
 (segment (start 127 55.88) (end 134.62 55.88) (width 0.2) (layer "B.Cu") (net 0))
 (segment (start 144.78 27.94) (end 137.16 27.94) (width 0.2) (layer "B.Cu") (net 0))
 (segment (start 137.16 27.94) (end 134.62 25.4) (width 0.2) (layer "B.Cu") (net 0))
 (segment (start 145.034 38.1) (end 139.7 38.1) (width 0.25) (layer "B.Cu") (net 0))
 (segment (start 134.62 68.58) (end 134.62 96.52) (width 0.25) (layer "B.Cu") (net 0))
 (segment (start 114.3 25.4) (end 134.62 25.4) (width 0.2) (layer "B.Cu") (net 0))
 (segment (start 139.7 38.1) (end 139.7 63.5) (width 0.25) (layer "B.Cu") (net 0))
 (segment (start 114.3 83.82) (end 114.3 86.36) (width 0.25) (layer "B.Cu") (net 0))
 (segment (start 73.66 66.04) (end 93.98 66.04) (width 0.2) (layer "B.Cu") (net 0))
 (segment (start 127 96.52) (end 134.62 96.52) (width 0.25) (layer "B.Cu") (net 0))
 (segment (start 145.034 33.02) (end 137.16 33.02) (width 0.2) (layer "B.Cu") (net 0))
 (segment (start 121.92 45.72) (end 114.3 45.72) (width 0.25) (layer "B.Cu") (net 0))
 (segment (start 83.82 106.68) (end 114.3 106.68) (width 0.25) (layer "B.Cu") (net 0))
 (segment (start 93.98 66.04) (end 114.3 66.04) (width 0.2) (layer "B.Cu") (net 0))
 (segment (start 73.66 86.36) (end 93.98 86.36) (width 0.25) (layer "B.Cu") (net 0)))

